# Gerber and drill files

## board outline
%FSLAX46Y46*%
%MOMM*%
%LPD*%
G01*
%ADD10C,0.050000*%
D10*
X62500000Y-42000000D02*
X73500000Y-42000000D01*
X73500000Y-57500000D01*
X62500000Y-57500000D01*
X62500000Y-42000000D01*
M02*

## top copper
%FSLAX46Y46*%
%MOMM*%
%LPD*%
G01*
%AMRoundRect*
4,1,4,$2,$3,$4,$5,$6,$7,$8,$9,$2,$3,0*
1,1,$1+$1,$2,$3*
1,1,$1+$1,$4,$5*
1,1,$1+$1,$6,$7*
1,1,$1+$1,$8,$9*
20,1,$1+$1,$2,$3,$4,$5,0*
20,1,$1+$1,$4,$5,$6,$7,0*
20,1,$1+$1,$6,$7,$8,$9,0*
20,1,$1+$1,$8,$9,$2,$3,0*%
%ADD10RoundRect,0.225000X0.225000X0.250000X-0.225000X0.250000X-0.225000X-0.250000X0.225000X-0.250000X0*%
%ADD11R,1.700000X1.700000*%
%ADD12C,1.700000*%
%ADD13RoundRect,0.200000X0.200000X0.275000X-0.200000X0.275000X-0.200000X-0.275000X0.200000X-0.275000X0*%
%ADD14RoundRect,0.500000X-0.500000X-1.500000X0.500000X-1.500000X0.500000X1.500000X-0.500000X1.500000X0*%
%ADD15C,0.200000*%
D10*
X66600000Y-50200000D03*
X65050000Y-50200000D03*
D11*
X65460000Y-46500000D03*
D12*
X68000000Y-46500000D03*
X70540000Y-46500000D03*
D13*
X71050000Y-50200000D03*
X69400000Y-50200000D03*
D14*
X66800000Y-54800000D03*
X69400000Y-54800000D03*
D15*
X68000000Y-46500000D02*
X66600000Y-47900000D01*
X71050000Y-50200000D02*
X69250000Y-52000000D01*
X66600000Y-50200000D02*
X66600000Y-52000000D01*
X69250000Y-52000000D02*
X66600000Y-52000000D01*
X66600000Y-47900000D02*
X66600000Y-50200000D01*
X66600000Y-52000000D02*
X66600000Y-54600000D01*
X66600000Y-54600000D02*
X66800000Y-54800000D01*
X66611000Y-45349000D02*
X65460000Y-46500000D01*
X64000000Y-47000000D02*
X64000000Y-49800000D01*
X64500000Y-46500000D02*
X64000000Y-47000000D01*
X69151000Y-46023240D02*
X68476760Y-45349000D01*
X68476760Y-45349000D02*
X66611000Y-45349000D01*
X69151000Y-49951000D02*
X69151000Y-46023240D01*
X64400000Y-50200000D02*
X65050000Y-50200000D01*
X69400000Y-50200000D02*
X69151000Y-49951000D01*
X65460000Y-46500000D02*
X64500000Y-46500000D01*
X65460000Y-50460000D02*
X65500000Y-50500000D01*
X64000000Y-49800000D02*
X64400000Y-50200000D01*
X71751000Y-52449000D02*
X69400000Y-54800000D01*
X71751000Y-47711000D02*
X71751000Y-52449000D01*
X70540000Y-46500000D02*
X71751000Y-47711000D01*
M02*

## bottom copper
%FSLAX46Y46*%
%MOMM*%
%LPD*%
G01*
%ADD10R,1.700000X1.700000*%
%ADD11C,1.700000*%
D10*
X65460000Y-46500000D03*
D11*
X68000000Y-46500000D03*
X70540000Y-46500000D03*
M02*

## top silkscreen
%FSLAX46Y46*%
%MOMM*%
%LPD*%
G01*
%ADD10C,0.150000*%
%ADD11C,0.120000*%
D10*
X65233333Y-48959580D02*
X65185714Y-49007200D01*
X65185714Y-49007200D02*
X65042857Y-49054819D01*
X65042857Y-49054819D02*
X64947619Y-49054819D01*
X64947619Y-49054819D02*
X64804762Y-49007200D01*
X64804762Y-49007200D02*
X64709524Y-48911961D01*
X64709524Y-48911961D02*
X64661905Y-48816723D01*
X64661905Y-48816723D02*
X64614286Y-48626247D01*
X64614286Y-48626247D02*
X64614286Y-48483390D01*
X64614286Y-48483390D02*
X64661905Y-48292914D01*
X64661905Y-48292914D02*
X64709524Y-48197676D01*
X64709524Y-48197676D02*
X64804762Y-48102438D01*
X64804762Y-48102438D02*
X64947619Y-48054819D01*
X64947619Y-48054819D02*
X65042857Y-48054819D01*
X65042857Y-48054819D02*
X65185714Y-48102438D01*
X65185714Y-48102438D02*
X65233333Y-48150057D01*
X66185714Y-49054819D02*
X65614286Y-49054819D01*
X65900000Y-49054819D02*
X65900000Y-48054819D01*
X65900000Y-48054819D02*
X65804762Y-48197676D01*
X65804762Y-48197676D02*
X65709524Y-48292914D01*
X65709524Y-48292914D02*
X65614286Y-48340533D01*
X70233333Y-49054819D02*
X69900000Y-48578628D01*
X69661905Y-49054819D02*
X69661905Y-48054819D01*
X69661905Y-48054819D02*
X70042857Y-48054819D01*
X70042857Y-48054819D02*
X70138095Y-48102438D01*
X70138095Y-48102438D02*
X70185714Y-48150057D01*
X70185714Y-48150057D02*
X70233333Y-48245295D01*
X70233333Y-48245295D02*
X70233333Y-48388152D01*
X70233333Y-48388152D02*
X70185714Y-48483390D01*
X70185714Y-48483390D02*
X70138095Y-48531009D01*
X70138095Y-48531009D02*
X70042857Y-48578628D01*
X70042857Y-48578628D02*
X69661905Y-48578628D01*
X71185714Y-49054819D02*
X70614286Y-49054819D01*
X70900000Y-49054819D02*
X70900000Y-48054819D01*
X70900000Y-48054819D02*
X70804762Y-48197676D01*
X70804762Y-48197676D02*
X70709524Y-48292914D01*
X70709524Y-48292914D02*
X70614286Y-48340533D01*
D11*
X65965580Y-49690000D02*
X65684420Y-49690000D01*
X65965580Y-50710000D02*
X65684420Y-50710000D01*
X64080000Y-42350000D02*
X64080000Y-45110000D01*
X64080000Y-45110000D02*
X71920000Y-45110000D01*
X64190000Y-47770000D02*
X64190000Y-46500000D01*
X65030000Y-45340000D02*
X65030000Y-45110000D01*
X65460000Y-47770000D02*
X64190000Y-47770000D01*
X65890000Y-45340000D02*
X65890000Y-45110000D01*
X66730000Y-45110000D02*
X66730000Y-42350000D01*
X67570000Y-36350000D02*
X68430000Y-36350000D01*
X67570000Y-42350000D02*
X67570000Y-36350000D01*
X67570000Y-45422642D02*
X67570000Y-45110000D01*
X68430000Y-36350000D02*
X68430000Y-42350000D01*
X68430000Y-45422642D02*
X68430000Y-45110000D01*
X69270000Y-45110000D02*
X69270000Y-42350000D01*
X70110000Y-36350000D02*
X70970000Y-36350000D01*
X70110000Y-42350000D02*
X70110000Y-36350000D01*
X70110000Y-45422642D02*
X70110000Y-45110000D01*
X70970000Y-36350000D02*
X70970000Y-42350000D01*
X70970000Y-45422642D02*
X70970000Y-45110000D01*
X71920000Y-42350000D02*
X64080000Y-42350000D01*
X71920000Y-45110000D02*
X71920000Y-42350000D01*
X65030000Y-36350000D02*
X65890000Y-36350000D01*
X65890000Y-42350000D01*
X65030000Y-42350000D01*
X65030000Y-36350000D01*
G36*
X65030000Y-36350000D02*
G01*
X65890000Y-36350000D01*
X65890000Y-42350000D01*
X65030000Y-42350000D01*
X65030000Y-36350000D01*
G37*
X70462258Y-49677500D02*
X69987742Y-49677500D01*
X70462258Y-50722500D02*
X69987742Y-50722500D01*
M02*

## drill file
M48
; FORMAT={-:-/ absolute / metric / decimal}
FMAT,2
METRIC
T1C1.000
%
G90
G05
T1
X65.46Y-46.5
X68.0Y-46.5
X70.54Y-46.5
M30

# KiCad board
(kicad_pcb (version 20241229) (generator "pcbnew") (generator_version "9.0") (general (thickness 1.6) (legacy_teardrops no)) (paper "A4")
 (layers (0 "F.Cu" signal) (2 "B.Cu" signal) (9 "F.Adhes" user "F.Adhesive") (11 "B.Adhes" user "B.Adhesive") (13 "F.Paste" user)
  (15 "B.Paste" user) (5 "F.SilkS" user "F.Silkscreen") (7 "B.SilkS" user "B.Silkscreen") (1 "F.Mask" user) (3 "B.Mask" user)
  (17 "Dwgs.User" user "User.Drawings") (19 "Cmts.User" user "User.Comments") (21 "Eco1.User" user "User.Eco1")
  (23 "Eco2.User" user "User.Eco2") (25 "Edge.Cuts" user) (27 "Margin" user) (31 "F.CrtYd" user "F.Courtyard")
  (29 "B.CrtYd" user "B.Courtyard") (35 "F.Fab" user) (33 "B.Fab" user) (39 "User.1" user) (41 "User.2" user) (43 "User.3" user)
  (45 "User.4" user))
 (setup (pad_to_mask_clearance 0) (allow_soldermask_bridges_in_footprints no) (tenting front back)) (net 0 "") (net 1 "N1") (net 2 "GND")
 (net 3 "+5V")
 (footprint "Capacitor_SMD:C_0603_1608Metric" (layer "F.Cu") (at 65.825 50.2 180)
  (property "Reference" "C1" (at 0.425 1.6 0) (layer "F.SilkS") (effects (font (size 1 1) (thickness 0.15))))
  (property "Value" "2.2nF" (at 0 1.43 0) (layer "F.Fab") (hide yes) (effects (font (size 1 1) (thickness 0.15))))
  (fp_line (start -0.14058 0.51) (end 0.14058 0.51) (stroke (width 0.12) (type solid)) (layer "F.SilkS"))
  (fp_line (start -0.14058 -0.51) (end 0.14058 -0.51) (stroke (width 0.12) (type solid)) (layer "F.SilkS"))
  (pad "1" smd roundrect (at -0.775 0 180) (size 0.9 0.95) (layers "F.Cu" "F.Mask" "F.Paste") (roundrect_rratio 0.25) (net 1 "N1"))
  (pad "2" smd roundrect (at 0.775 0 180) (size 0.9 0.95) (layers "F.Cu" "F.Mask" "F.Paste") (roundrect_rratio 0.25) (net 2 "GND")))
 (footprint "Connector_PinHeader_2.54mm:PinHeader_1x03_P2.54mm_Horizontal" (layer "F.Cu") (at 65.46 46.5 90)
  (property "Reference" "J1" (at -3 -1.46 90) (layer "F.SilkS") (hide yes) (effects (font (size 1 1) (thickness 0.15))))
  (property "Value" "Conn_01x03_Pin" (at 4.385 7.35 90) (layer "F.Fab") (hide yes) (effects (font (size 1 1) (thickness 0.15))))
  (fp_line (start 4.15 -1.38) (end 1.39 -1.38) (stroke (width 0.12) (type solid)) (layer "F.SilkS"))
  (fp_line (start 1.39 -1.38) (end 1.39 6.46) (stroke (width 0.12) (type solid)) (layer "F.SilkS"))
  (fp_line (start -1.27 -1.27) (end 0 -1.27) (stroke (width 0.12) (type solid)) (layer "F.SilkS"))
  (fp_line (start 1.16 -0.43) (end 1.39 -0.43) (stroke (width 0.12) (type solid)) (layer "F.SilkS"))
  (fp_line (start -1.27 0) (end -1.27 -1.27) (stroke (width 0.12) (type solid)) (layer "F.SilkS"))
  (fp_line (start 1.16 0.43) (end 1.39 0.43) (stroke (width 0.12) (type solid)) (layer "F.SilkS"))
  (fp_line (start 1.39 1.27) (end 4.15 1.27) (stroke (width 0.12) (type solid)) (layer "F.SilkS"))
  (fp_line (start 10.15 2.11) (end 10.15 2.97) (stroke (width 0.12) (type solid)) (layer "F.SilkS"))
  (fp_line (start 4.15 2.11) (end 10.15 2.11) (stroke (width 0.12) (type solid)) (layer "F.SilkS"))
  (fp_line (start 1.077358 2.11) (end 1.39 2.11) (stroke (width 0.12) (type solid)) (layer "F.SilkS"))
  (fp_line (start 10.15 2.97) (end 4.15 2.97) (stroke (width 0.12) (type solid)) (layer "F.SilkS"))
  (fp_line (start 1.077358 2.97) (end 1.39 2.97) (stroke (width 0.12) (type solid)) (layer "F.SilkS"))
  (fp_line (start 1.39 3.81) (end 4.15 3.81) (stroke (width 0.12) (type solid)) (layer "F.SilkS"))
  (fp_line (start 10.15 4.65) (end 10.15 5.51) (stroke (width 0.12) (type solid)) (layer "F.SilkS"))
  (fp_line (start 4.15 4.65) (end 10.15 4.65) (stroke (width 0.12) (type solid)) (layer "F.SilkS"))
  (fp_line (start 1.077358 4.65) (end 1.39 4.65) (stroke (width 0.12) (type solid)) (layer "F.SilkS"))
  (fp_line (start 10.15 5.51) (end 4.15 5.51) (stroke (width 0.12) (type solid)) (layer "F.SilkS"))
  (fp_line (start 1.077358 5.51) (end 1.39 5.51) (stroke (width 0.12) (type solid)) (layer "F.SilkS"))
  (fp_line (start 4.15 6.46) (end 4.15 -1.38) (stroke (width 0.12) (type solid)) (layer "F.SilkS"))
  (fp_line (start 1.39 6.46) (end 4.15 6.46) (stroke (width 0.12) (type solid)) (layer "F.SilkS"))
  (fp_rect (start 4.15 -0.43) (end 10.15 0.43) (stroke (width 0.12) (type solid)) (fill yes) (layer "F.SilkS"))
  (pad "1" thru_hole rect (at 0 0 90) (size 1.7 1.7) (drill 1) (layers "*.Cu" "*.Mask") (remove_unused_layers no) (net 2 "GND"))
  (pad "2" thru_hole circle (at 0 2.54 90) (size 1.7 1.7) (drill 1) (layers "*.Cu" "*.Mask") (remove_unused_layers no) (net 1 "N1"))
  (pad "3" thru_hole circle (at 0 5.08 90) (size 1.7 1.7) (drill 1) (layers "*.Cu" "*.Mask") (remove_unused_layers no) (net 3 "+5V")))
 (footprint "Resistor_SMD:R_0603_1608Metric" (layer "F.Cu") (at 70.225 50.2 180)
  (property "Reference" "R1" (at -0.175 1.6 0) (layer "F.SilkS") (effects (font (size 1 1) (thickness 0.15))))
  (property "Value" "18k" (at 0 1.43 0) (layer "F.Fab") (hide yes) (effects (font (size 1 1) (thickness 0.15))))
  (fp_line (start -0.237258 0.5225) (end 0.237258 0.5225) (stroke (width 0.12) (type solid)) (layer "F.SilkS"))
  (fp_line (start -0.237258 -0.5225) (end 0.237258 -0.5225) (stroke (width 0.12) (type solid)) (layer "F.SilkS"))
  (pad "1" smd roundrect (at -0.825 0 180) (size 0.8 0.95) (layers "F.Cu" "F.Mask" "F.Paste") (roundrect_rratio 0.25) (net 1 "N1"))
  (pad "2" smd roundrect (at 0.825 0 180) (size 0.8 0.95) (layers "F.Cu" "F.Mask" "F.Paste") (roundrect_rratio 0.25) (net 2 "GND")))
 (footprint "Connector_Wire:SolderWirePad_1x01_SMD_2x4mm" (layer "F.Cu") (at 66.8 54.8)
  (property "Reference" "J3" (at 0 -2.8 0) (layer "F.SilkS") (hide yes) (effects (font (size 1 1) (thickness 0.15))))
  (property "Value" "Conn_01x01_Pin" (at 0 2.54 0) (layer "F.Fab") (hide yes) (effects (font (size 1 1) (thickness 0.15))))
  (pad "1" smd roundrect (at 0 0) (size 2 4) (layers "F.Cu" "F.Mask") (roundrect_rratio 0.25) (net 1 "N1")))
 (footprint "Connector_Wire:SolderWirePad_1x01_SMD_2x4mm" (layer "F.Cu") (at 69.4 54.8)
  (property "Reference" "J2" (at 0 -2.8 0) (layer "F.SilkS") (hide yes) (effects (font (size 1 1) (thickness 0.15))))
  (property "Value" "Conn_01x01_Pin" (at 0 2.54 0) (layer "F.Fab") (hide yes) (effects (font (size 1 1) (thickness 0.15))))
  (pad "1" smd roundrect (at 0 0) (size 2 4) (layers "F.Cu" "F.Mask") (roundrect_rratio 0.25) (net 3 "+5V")))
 (gr_rect (start 62.5 42) (end 73.5 57.5) (stroke (width 0.05) (type default)) (fill no) (layer "Edge.Cuts"))
 (segment (start 68 46.5) (end 66.6 47.9) (width 0.2) (layer "F.Cu") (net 1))
 (segment (start 71.05 50.2) (end 69.25 52) (width 0.2) (layer "F.Cu") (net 1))
 (segment (start 66.6 50.2) (end 66.6 52) (width 0.2) (layer "F.Cu") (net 1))
 (segment (start 69.25 52) (end 66.6 52) (width 0.2) (layer "F.Cu") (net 1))
 (segment (start 66.6 47.9) (end 66.6 50.2) (width 0.2) (layer "F.Cu") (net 1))
 (segment (start 66.6 52) (end 66.6 54.6) (width 0.2) (layer "F.Cu") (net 1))
 (segment (start 66.6 54.6) (end 66.8 54.8) (width 0.2) (layer "F.Cu") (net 1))
 (segment (start 66.611 45.349) (end 65.46 46.5) (width 0.2) (layer "F.Cu") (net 2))
 (segment (start 64 47) (end 64 49.8) (width 0.2) (layer "F.Cu") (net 2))
 (segment (start 64.5 46.5) (end 64 47) (width 0.2) (layer "F.Cu") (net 2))
 (segment (start 69.151 46.02324) (end 68.47676 45.349) (width 0.2) (layer "F.Cu") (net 2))
 (segment (start 68.47676 45.349) (end 66.611 45.349) (width 0.2) (layer "F.Cu") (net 2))
 (segment (start 69.151 49.951) (end 69.151 46.02324) (width 0.2) (layer "F.Cu") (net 2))
 (segment (start 64.4 50.2) (end 65.05 50.2) (width 0.2) (layer "F.Cu") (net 2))
 (segment (start 69.4 50.2) (end 69.151 49.951) (width 0.2) (layer "F.Cu") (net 2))
 (segment (start 65.46 46.5) (end 64.5 46.5) (width 0.2) (layer "F.Cu") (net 2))
 (segment (start 65.46 50.46) (end 65.5 50.5) (width 0.2) (layer "F.Cu") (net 2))
 (segment (start 64 49.8) (end 64.4 50.2) (width 0.2) (layer "F.Cu") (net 2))
 (segment (start 71.751 52.449) (end 69.4 54.8) (width 0.2) (layer "F.Cu") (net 3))
 (segment (start 71.751 47.711) (end 71.751 52.449) (width 0.2) (layer "F.Cu") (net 3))
 (segment (start 70.54 46.5) (end 71.751 47.711) (width 0.2) (layer "F.Cu") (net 3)))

